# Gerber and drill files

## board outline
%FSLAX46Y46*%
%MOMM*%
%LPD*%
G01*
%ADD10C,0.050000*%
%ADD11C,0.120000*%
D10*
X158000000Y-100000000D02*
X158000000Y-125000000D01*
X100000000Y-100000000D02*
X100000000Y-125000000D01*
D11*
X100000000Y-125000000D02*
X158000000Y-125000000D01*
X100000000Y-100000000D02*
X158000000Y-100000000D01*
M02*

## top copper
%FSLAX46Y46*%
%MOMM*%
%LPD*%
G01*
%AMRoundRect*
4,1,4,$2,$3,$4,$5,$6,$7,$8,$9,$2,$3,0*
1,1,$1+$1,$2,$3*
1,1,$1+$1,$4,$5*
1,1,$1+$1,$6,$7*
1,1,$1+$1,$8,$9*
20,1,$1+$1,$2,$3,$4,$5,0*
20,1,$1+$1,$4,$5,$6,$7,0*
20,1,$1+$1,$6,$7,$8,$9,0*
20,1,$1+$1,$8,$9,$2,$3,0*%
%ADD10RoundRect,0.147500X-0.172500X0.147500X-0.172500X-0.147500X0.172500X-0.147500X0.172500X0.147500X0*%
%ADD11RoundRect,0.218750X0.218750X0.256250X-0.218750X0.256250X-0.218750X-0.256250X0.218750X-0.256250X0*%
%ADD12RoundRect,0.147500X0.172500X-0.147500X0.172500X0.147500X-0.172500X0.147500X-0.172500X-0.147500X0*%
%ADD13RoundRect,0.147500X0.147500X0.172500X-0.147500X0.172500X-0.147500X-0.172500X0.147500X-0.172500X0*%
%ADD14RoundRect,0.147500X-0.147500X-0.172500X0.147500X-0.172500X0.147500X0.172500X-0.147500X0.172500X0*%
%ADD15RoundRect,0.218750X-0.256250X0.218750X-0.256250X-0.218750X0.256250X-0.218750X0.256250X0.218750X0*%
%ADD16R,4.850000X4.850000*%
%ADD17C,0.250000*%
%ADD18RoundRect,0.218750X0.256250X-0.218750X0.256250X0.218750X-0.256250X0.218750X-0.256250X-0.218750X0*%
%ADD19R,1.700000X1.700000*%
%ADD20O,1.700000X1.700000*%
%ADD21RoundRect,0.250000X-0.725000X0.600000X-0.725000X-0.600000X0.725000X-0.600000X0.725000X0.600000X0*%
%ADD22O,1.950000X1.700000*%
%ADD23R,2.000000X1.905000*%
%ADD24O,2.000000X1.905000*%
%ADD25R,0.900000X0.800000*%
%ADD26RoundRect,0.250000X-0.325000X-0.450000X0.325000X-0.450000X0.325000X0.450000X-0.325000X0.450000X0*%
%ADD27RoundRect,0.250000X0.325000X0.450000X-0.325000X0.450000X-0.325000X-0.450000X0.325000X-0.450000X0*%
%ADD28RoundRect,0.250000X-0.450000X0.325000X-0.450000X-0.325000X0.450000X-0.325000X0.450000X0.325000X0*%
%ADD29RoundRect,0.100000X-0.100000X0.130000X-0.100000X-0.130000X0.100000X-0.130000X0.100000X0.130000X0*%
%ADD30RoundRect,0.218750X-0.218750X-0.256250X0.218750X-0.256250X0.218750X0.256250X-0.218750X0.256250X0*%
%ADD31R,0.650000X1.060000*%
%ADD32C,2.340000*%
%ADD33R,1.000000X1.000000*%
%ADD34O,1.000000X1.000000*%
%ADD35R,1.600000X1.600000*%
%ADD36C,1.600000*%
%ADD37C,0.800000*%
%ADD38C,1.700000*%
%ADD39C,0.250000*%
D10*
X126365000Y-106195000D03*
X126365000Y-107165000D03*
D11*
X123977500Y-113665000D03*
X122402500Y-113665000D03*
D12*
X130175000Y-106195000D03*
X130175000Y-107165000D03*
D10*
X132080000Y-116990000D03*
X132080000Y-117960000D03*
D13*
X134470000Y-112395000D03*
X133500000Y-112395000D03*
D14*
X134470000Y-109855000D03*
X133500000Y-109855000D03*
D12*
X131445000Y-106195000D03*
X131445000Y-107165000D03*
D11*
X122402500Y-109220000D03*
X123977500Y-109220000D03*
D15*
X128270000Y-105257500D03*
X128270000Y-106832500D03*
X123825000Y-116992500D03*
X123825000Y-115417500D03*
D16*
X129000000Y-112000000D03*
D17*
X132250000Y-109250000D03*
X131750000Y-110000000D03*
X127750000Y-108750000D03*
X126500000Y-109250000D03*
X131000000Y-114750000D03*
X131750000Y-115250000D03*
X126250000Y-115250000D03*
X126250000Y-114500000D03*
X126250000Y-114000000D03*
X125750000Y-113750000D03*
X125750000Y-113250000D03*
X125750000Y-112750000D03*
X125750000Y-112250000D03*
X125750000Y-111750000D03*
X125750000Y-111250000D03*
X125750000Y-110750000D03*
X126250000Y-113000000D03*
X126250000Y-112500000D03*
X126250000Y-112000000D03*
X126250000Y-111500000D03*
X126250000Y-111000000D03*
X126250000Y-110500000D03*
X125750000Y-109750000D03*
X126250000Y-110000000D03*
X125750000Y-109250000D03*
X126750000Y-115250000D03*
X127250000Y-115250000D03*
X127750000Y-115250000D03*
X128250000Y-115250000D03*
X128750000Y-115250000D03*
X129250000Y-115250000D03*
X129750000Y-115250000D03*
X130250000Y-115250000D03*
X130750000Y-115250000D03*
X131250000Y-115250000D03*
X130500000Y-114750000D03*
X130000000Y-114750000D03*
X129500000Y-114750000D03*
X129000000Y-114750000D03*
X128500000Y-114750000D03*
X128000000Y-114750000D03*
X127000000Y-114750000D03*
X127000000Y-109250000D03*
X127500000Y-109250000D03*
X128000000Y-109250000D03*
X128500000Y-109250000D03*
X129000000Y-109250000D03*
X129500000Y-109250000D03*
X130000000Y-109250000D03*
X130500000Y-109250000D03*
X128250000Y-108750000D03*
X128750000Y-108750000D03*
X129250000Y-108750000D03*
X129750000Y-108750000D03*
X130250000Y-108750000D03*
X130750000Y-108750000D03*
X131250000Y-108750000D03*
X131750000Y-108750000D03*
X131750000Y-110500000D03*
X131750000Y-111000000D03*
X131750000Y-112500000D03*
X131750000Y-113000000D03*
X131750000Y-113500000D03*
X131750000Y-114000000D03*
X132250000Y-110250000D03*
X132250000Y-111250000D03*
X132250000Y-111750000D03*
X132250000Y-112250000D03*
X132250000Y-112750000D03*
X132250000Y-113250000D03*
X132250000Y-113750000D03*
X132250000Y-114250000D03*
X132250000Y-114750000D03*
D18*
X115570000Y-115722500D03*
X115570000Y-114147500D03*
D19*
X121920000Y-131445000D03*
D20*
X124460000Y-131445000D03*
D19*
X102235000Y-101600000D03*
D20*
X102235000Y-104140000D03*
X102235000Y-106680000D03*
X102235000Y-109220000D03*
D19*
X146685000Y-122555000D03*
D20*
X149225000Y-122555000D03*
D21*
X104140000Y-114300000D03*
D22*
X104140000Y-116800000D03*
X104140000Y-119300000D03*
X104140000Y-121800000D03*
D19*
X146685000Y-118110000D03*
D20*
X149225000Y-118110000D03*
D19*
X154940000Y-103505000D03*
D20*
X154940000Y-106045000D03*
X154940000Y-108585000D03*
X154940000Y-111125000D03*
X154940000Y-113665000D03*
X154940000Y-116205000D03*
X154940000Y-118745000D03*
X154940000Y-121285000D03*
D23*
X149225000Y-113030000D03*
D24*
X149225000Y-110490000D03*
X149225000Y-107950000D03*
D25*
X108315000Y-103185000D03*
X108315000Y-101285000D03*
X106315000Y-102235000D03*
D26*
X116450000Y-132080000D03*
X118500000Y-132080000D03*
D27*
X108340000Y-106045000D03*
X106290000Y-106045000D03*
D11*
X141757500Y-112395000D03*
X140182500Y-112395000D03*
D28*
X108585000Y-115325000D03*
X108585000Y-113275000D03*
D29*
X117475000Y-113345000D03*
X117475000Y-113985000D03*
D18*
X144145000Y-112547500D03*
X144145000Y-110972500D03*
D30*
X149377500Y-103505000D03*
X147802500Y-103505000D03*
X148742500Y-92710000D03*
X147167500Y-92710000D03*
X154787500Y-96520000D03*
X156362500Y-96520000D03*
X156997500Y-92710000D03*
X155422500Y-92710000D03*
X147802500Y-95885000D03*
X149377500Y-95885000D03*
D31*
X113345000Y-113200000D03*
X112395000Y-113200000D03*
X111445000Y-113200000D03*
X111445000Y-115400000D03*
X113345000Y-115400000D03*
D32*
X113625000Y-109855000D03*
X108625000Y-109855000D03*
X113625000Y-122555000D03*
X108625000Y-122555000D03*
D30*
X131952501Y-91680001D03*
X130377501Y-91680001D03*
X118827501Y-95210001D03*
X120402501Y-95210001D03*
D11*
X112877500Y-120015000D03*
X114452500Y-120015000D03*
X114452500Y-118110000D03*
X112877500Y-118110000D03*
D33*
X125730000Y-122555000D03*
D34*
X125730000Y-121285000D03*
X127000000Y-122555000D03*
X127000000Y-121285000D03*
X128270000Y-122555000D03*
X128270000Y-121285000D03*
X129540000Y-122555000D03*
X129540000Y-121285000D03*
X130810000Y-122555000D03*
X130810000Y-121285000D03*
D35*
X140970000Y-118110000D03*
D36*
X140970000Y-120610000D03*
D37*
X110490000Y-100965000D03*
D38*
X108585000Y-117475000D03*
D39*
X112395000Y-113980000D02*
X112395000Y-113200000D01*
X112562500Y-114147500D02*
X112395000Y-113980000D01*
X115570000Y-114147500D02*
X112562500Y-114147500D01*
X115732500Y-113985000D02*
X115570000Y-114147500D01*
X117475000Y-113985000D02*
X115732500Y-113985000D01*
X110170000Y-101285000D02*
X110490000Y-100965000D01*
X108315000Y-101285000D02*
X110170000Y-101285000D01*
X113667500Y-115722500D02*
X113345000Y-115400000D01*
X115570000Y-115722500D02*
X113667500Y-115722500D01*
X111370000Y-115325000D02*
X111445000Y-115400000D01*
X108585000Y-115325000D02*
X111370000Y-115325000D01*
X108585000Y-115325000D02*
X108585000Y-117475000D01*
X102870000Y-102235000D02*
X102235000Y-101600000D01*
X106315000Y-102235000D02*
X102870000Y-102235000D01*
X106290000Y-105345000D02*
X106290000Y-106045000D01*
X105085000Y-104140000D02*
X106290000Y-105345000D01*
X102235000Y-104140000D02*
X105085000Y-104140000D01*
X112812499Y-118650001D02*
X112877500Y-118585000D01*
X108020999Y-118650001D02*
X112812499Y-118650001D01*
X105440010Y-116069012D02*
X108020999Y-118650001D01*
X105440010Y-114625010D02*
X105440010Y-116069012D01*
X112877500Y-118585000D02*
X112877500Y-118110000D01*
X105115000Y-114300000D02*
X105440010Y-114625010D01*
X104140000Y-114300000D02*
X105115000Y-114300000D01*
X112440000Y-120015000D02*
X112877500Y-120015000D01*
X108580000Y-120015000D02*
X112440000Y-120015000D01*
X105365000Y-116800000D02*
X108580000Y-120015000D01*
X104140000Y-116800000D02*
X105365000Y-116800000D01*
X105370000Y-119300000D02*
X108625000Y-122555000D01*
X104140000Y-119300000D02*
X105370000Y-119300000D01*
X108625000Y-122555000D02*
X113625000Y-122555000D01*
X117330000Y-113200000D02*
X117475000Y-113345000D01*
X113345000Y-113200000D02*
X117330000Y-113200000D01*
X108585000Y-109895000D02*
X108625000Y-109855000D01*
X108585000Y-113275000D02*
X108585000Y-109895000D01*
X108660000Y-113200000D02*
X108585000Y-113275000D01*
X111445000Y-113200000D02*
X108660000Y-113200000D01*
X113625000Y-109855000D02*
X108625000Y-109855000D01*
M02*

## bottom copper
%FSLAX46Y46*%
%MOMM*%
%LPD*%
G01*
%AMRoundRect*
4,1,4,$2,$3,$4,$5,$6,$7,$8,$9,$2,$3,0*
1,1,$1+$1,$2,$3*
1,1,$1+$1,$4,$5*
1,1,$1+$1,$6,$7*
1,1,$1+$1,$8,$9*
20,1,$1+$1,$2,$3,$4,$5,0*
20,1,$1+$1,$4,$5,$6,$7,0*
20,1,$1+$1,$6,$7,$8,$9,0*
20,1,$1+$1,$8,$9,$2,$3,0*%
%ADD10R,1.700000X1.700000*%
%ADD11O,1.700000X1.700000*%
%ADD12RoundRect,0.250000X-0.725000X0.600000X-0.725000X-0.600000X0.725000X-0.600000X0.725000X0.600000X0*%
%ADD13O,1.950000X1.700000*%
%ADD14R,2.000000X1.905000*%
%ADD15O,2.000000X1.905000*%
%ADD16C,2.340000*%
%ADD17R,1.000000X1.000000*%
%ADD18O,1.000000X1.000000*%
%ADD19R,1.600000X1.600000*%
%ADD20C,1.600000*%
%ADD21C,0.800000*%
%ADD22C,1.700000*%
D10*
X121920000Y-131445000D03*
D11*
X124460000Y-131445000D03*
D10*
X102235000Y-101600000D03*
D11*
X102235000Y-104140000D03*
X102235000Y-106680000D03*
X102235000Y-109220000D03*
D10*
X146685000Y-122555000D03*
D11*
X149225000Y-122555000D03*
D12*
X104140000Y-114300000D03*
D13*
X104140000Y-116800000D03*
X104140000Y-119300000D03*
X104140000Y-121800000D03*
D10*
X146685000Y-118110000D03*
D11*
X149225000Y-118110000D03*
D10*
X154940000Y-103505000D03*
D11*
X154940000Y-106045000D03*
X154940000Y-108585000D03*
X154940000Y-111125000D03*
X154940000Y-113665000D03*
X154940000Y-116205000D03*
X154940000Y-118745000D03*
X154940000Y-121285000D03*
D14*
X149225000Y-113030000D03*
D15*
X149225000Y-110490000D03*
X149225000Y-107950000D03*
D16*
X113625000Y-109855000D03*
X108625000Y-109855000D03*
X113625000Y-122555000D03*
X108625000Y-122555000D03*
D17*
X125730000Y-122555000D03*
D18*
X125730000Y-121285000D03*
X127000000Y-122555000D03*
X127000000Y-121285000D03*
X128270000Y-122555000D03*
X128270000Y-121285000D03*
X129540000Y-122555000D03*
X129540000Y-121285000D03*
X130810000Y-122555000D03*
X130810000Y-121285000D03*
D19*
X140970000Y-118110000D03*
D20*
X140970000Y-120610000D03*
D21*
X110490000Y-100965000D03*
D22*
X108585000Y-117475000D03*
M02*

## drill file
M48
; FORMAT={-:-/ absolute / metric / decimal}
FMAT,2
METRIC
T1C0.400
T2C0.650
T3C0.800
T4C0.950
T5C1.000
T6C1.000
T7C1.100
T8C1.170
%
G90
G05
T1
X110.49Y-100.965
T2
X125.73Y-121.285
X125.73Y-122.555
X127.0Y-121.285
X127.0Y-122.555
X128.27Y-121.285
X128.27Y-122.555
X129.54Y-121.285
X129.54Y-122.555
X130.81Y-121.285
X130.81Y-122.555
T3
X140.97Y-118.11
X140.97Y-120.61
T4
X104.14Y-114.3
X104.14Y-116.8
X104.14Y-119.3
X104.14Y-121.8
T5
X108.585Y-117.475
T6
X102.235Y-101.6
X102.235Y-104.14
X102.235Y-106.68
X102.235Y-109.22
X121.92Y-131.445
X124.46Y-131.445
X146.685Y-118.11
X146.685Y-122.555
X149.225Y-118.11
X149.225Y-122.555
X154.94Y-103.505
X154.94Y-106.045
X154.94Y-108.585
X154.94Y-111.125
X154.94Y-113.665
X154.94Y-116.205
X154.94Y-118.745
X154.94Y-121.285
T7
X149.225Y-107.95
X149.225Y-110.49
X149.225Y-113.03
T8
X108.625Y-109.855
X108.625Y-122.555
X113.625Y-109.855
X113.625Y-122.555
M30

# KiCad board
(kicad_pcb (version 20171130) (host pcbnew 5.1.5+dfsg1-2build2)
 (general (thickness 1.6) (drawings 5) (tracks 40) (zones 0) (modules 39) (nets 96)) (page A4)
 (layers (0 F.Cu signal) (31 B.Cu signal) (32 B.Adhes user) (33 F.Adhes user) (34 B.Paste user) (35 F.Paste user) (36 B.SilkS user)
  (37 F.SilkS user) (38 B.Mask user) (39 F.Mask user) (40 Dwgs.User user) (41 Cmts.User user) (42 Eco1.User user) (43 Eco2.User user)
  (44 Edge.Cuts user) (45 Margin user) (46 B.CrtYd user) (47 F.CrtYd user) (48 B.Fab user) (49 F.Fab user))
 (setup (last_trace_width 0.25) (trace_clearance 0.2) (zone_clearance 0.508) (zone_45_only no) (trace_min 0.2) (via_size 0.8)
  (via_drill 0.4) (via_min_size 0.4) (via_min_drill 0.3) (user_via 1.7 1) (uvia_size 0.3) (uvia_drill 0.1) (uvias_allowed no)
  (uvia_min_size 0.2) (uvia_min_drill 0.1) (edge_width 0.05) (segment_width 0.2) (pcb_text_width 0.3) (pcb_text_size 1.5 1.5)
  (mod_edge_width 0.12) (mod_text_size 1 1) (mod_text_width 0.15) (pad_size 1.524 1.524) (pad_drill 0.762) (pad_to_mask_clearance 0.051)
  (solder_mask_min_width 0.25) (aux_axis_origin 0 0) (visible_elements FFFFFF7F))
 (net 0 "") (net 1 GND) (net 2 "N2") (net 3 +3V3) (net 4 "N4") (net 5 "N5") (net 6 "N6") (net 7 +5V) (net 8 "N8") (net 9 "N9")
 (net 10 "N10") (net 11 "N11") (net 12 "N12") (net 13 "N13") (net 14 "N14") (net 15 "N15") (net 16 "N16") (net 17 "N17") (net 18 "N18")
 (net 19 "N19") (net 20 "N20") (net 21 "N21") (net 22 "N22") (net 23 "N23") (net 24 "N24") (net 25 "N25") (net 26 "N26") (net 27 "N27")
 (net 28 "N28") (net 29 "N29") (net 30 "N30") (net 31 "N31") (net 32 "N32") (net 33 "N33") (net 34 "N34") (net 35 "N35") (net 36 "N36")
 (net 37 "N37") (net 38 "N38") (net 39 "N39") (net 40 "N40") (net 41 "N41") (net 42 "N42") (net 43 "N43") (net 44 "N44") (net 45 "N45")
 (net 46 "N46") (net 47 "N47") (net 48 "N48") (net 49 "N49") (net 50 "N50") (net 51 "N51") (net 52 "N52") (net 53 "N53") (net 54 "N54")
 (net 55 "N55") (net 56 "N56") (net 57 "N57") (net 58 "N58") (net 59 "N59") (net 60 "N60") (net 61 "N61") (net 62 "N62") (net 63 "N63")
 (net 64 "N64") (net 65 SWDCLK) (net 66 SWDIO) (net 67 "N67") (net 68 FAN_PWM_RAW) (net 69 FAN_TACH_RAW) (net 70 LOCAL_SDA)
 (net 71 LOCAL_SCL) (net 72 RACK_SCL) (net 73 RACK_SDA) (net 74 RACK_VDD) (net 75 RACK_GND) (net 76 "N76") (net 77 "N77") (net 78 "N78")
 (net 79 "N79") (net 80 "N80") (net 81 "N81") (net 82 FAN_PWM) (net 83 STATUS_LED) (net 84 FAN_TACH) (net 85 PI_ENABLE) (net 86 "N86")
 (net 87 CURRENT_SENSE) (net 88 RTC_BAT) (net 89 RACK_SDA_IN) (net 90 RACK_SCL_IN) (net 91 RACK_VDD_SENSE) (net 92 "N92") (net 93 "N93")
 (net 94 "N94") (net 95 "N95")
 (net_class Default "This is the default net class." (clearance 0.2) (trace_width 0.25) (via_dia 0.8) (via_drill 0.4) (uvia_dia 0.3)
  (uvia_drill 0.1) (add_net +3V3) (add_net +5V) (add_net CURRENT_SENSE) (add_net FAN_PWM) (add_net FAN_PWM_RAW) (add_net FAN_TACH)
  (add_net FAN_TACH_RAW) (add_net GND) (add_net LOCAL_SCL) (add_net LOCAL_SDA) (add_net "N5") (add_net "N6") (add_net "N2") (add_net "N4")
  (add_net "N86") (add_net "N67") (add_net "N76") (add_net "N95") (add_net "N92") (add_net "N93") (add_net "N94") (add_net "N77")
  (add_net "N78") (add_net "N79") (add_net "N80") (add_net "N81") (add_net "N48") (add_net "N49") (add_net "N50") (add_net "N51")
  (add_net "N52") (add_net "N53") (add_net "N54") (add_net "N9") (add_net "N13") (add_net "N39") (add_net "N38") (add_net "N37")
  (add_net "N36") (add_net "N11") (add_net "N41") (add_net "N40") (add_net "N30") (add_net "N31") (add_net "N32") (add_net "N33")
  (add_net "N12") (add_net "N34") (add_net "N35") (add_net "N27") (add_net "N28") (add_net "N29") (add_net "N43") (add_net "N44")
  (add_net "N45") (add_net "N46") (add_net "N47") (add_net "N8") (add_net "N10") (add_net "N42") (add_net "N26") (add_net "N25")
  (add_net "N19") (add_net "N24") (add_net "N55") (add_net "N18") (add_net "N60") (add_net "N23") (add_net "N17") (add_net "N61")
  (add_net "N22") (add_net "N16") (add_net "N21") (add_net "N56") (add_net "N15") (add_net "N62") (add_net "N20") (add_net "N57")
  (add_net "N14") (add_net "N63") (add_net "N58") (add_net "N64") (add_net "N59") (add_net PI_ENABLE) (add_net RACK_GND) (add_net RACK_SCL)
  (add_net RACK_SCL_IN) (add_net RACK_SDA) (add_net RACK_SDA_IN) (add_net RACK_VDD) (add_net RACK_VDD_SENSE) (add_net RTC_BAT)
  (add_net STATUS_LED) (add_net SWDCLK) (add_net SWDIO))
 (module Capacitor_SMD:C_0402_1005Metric (layer F.Cu) (at 126.365 106.68 270)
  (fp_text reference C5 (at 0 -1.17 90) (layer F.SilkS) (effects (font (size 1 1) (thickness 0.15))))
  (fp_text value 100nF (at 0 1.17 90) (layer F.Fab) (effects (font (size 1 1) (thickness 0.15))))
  (pad 1 smd roundrect (at -0.485 0 270) (size 0.59 0.64) (layers F.Cu F.Paste F.Mask) (roundrect_rratio 0.25) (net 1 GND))
  (pad 2 smd roundrect (at 0.485 0 270) (size 0.59 0.64) (layers F.Cu F.Paste F.Mask) (roundrect_rratio 0.25) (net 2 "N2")))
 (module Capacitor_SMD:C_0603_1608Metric (layer F.Cu) (at 123.19 113.665 180)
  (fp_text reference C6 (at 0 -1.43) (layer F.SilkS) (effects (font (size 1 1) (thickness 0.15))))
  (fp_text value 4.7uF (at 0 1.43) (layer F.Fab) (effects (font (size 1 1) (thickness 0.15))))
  (pad 1 smd roundrect (at -0.7875 0 180) (size 0.875 0.95) (layers F.Cu F.Paste F.Mask) (roundrect_rratio 0.25) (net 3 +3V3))
  (pad 2 smd roundrect (at 0.7875 0 180) (size 0.875 0.95) (layers F.Cu F.Paste F.Mask) (roundrect_rratio 0.25) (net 1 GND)))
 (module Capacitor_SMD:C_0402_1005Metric (layer F.Cu) (at 130.175 106.68 90)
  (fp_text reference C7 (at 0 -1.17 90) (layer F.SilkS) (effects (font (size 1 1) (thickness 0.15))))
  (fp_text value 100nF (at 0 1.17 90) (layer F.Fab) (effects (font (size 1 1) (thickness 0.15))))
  (pad 2 smd roundrect (at 0.485 0 90) (size 0.59 0.64) (layers F.Cu F.Paste F.Mask) (roundrect_rratio 0.25) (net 1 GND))
  (pad 1 smd roundrect (at -0.485 0 90) (size 0.59 0.64) (layers F.Cu F.Paste F.Mask) (roundrect_rratio 0.25) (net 3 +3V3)))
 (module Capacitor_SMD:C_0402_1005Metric (layer F.Cu) (at 132.08 117.475 270)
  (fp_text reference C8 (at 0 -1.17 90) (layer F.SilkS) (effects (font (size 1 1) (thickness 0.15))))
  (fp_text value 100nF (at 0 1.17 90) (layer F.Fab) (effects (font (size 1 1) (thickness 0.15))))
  (pad 1 smd roundrect (at -0.485 0 270) (size 0.59 0.64) (layers F.Cu F.Paste F.Mask) (roundrect_rratio 0.25) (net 3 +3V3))
  (pad 2 smd roundrect (at 0.485 0 270) (size 0.59 0.64) (layers F.Cu F.Paste F.Mask) (roundrect_rratio 0.25) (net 1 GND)))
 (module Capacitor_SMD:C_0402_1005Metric (layer F.Cu) (at 133.985 112.395 180)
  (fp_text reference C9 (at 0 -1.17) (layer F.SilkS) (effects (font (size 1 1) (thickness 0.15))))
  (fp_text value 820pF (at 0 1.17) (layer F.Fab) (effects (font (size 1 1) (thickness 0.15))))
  (pad 1 smd roundrect (at -0.485 0 180) (size 0.59 0.64) (layers F.Cu F.Paste F.Mask) (roundrect_rratio 0.25) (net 1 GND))
  (pad 2 smd roundrect (at 0.485 0 180) (size 0.59 0.64) (layers F.Cu F.Paste F.Mask) (roundrect_rratio 0.25) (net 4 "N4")))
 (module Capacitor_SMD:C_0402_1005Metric (layer F.Cu) (at 133.985 109.855)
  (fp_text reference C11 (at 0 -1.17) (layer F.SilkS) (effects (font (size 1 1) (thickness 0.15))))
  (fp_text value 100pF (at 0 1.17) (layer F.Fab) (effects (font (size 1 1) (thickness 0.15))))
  (pad 2 smd roundrect (at 0.485 0) (size 0.59 0.64) (layers F.Cu F.Paste F.Mask) (roundrect_rratio 0.25) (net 1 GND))
  (pad 1 smd roundrect (at -0.485 0) (size 0.59 0.64) (layers F.Cu F.Paste F.Mask) (roundrect_rratio 0.25) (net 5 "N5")))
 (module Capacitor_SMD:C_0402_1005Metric (layer F.Cu) (at 131.445 106.68 90)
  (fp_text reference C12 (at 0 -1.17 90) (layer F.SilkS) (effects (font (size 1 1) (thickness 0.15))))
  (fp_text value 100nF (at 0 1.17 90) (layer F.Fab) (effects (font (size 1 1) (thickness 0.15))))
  (pad 2 smd roundrect (at 0.485 0 90) (size 0.59 0.64) (layers F.Cu F.Paste F.Mask) (roundrect_rratio 0.25) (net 1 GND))
  (pad 1 smd roundrect (at -0.485 0 90) (size 0.59 0.64) (layers F.Cu F.Paste F.Mask) (roundrect_rratio 0.25) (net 3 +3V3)))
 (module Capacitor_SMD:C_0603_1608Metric (layer F.Cu) (at 123.19 109.22 180)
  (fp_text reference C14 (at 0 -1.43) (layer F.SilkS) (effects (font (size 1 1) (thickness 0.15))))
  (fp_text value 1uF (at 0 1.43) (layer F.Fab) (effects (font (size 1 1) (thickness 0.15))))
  (pad 2 smd roundrect (at 0.7875 0 180) (size 0.875 0.95) (layers F.Cu F.Paste F.Mask) (roundrect_rratio 0.25) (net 1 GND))
  (pad 1 smd roundrect (at -0.7875 0 180) (size 0.875 0.95) (layers F.Cu F.Paste F.Mask) (roundrect_rratio 0.25) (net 3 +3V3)))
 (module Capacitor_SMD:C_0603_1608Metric (layer F.Cu) (at 128.27 106.045 270)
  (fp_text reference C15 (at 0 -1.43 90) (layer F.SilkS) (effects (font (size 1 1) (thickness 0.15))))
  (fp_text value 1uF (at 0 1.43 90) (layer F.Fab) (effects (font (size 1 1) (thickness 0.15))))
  (pad 1 smd roundrect (at -0.7875 0 270) (size 0.875 0.95) (layers F.Cu F.Paste F.Mask) (roundrect_rratio 0.25) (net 1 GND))
  (pad 2 smd roundrect (at 0.7875 0 270) (size 0.875 0.95) (layers F.Cu F.Paste F.Mask) (roundrect_rratio 0.25) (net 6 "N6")))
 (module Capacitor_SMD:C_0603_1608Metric (layer F.Cu) (at 123.825 116.205 270)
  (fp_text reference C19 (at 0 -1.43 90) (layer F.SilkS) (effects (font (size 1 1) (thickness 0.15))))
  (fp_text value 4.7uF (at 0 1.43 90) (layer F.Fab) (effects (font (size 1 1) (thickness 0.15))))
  (pad 2 smd roundrect (at 0.7875 0 270) (size 0.875 0.95) (layers F.Cu F.Paste F.Mask) (roundrect_rratio 0.25) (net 1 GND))
  (pad 1 smd roundrect (at -0.7875 0 270) (size 0.875 0.95) (layers F.Cu F.Paste F.Mask) (roundrect_rratio 0.25) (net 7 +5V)))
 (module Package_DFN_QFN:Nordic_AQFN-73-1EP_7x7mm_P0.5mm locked (layer F.Cu) (at 129 112)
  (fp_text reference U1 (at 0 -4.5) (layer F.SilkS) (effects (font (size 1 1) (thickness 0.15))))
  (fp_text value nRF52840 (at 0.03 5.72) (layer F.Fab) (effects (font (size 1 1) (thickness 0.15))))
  (pad "" smd rect (at 1.2125 1.2125 180) (size 2 2) (layers F.Paste))
  (pad "" smd rect (at -1.2125 1.2125 180) (size 2 2) (layers F.Paste))
  (pad "" smd rect (at 1.2125 -1.2125 180) (size 2 2) (layers F.Paste))
  (pad "" smd rect (at -1.2125 -1.2125 180) (size 2 2) (layers F.Paste))
  (pad EP smd rect (at 0 0 180) (size 4.85 4.85) (layers F.Cu F.Mask) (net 1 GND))
  (pad B24 smd circle (at 3.25 -2.75 180) (size 0.25 0.25) (layers F.Cu F.Paste F.Mask) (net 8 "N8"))
  (pad D23 smd circle (at 2.75 -2 180) (size 0.25 0.25) (layers F.Cu F.Paste F.Mask) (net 5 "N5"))
  (pad A8 smd circle (at -1.25 -3.25 180) (size 0.25 0.25) (layers F.Cu F.Paste F.Mask) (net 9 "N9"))
  (pad B3 smd circle (at -2.5 -2.75 180) (size 0.25 0.25) (layers F.Cu F.Paste F.Mask) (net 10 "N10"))
  (pad AC21 smd circle (at 2 2.75 180) (size 0.25 0.25) (layers F.Cu F.Paste F.Mask) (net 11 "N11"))
  (pad AD23 smd circle (at 2.75 3.25 180) (size 0.25 0.25) (layers F.Cu F.Paste F.Mask) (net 3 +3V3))
  (pad AD2 smd circle (at -2.75 3.25 180) (size 0.25 0.25) (layers F.Cu F.Paste F.Mask) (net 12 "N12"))
  (pad AB2 smd circle (at -2.75 2.5 180) (size 0.25 0.25) (layers F.Cu F.Paste F.Mask) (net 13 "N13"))
  (pad Y2 smd circle (at -2.75 2 180) (size 0.25 0.25) (layers F.Cu F.Paste F.Mask) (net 7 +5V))
  (pad W1 smd circle (at -3.25 1.75 180) (size 0.25 0.25) (layers F.Cu F.Paste F.Mask) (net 3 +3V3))
  (pad U1 smd circle (at -3.25 1.25 180) (size 0.25 0.25) (layers F.Cu F.Paste F.Mask) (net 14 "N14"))
  (pad R1 smd circle (at -3.25 0.75 180) (size 0.25 0.25) (layers F.Cu F.Paste F.Mask) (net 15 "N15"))
  (pad N1 smd circle (at -3.25 0.25 180) (size 0.25 0.25) (layers F.Cu F.Paste F.Mask) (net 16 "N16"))
  (pad L1 smd circle (at -3.25 -0.25 180) (size 0.25 0.25) (layers F.Cu F.Paste F.Mask) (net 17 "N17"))
  (pad J1 smd circle (at -3.25 -0.75 180) (size 0.25 0.25) (layers F.Cu F.Paste F.Mask) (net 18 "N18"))
  (pad G1 smd circle (at -3.25 -1.25 180) (size 0.25 0.25) (layers F.Cu F.Paste F.Mask) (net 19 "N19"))
  (pad T2 smd circle (at -2.75 1 180) (size 0.25 0.25) (layers F.Cu F.Paste F.Mask) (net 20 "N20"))
  (pad P2 smd circle (at -2.75 0.5 180) (size 0.25 0.25) (layers F.Cu F.Paste F.Mask) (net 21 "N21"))
  (pad M2 smd circle (at -2.75 0 180) (size 0.25 0.25) (layers F.Cu F.Paste F.Mask) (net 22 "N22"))
  (pad K2 smd circle (at -2.75 -0.5 180) (size 0.25 0.25) (layers F.Cu F.Paste F.Mask) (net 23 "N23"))
  (pad H2 smd circle (at -2.75 -1 180) (size 0.25 0.25) (layers F.Cu F.Paste F.Mask) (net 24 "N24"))
  (pad F2 smd circle (at -2.75 -1.5 180) (size 0.25 0.25) (layers F.Cu F.Paste F.Mask) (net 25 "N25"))
  (pad C1 smd circle (at -3.25 -2.25 180) (size 0.25 0.25) (layers F.Cu F.Paste F.Mask) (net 2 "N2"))
  (pad D2 smd circle (at -2.75 -2 180) (size 0.25 0.25) (layers F.Cu F.Paste F.Mask) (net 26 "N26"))
  (pad B1 smd circle (at -3.25 -2.75 180) (size 0.25 0.25) (layers F.Cu F.Paste F.Mask) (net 3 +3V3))
  (pad AD4 smd circle (at -2.25 3.25 180) (size 0.25 0.25) (layers F.Cu F.Paste F.Mask) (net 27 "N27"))
  (pad AD6 smd circle (at -1.75 3.25 180) (size 0.25 0.25) (layers F.Cu F.Paste F.Mask) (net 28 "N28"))
  (pad AD8 smd circle (at -1.25 3.25 180) (size 0.25 0.25) (layers F.Cu F.Paste F.Mask) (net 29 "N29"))
  (pad AD10 smd circle (at -0.75 3.25 180) (size 0.25 0.25) (layers F.Cu F.Paste F.Mask) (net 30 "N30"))
  (pad AD12 smd circle (at -0.25 3.25 180) (size 0.25 0.25) (layers F.Cu F.Paste F.Mask) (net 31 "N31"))
  (pad AD14 smd circle (at 0.25 3.25 180) (size 0.25 0.25) (layers F.Cu F.Paste F.Mask) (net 3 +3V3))
  (pad AD16 smd circle (at 0.75 3.25 180) (size 0.25 0.25) (layers F.Cu F.Paste F.Mask) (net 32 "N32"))
  (pad AD18 smd circle (at 1.25 3.25 180) (size 0.25 0.25) (layers F.Cu F.Paste F.Mask) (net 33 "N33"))
  (pad AD20 smd circle (at 1.75 3.25 180) (size 0.25 0.25) (layers F.Cu F.Paste F.Mask) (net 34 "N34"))
  (pad AD22 smd circle (at 2.25 3.25 180) (size 0.25 0.25) (layers F.Cu F.Paste F.Mask) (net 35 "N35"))
  (pad AC19 smd circle (at 1.5 2.75 180) (size 0.25 0.25) (layers F.Cu F.Paste F.Mask) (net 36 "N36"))
  (pad AC17 smd circle (at 1 2.75 180) (size 0.25 0.25) (layers F.Cu F.Paste F.Mask) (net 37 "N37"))
  (pad AC15 smd circle (at 0.5 2.75 180) (size 0.25 0.25) (layers F.Cu F.Paste F.Mask) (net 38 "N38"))
  (pad AC13 smd circle (at 0 2.75 180) (size 0.25 0.25) (layers F.Cu F.Paste F.Mask) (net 3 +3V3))
  (pad AC11 smd circle (at -0.5 2.75 180) (size 0.25 0.25) (layers F.Cu F.Paste F.Mask) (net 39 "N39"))
  (pad AC9 smd circle (at -1 2.75 180) (size 0.25 0.25) (layers F.Cu F.Paste F.Mask) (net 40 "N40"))
  (pad AC5 smd circle (at -2 2.75 180) (size 0.25 0.25) (layers F.Cu F.Paste F.Mask) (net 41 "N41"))
  (pad B5 smd circle (at -2 -2.75 180) (size 0.25 0.25) (layers F.Cu F.Paste F.Mask) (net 6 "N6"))
  (pad B7 smd circle (at -1.5 -2.75 180) (size 0.25 0.25) (layers F.Cu F.Paste F.Mask) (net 1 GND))
  (pad B9 smd circle (at -1 -2.75 180) (size 0.25 0.25) (layers F.Cu F.Paste F.Mask) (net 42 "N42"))
  (pad B11 smd circle (at -0.5 -2.75 180) (size 0.25 0.25) (layers F.Cu F.Paste F.Mask) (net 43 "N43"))
  (pad B13 smd circle (at 0 -2.75 180) (size 0.25 0.25) (layers F.Cu F.Paste F.Mask) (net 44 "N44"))
  (pad B15 smd circle (at 0.5 -2.75 180) (size 0.25 0.25) (layers F.Cu F.Paste F.Mask) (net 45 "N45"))
  (pad B17 smd circle (at 1 -2.75 180) (size 0.25 0.25) (layers F.Cu F.Paste F.Mask) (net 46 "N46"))
  (pad B19 smd circle (at 1.5 -2.75 180) (size 0.25 0.25) (layers F.Cu F.Paste F.Mask) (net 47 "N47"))
  (pad A10 smd circle (at -0.75 -3.25 180) (size 0.25 0.25) (layers F.Cu F.Paste F.Mask) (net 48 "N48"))
  (pad A12 smd circle (at -0.25 -3.25 180) (size 0.25 0.25) (layers F.Cu F.Paste F.Mask) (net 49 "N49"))
  (pad A14 smd circle (at 0.25 -3.25 180) (size 0.25 0.25) (layers F.Cu F.Paste F.Mask) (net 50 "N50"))
  (pad A16 smd circle (at 0.75 -3.25 180) (size 0.25 0.25) (layers F.Cu F.Paste F.Mask) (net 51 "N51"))
  (pad A18 smd circle (at 1.25 -3.25 180) (size 0.25 0.25) (layers F.Cu F.Paste F.Mask) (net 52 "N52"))
  (pad A20 smd circle (at 1.75 -3.25 180) (size 0.25 0.25) (layers F.Cu F.Paste F.Mask) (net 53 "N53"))
  (pad A22 smd circle (at 2.25 -3.25 180) (size 0.25 0.25) (layers F.Cu F.Paste F.Mask) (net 3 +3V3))
  (pad A23 smd circle (at 2.75 -3.25 180) (size 0.25 0.25) (layers F.Cu F.Paste F.Mask) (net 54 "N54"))
  (pad F23 smd circle (at 2.75 -1.5 180) (size 0.25 0.25) (layers F.Cu F.Paste F.Mask) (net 1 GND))
  (pad H23 smd circle (at 2.75 -1 180) (size 0.25 0.25) (layers F.Cu F.Paste F.Mask) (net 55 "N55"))
  (pad P23 smd circle (at 2.75 0.5 180) (size 0.25 0.25) (layers F.Cu F.Paste F.Mask) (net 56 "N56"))
  (pad T23 smd circle (at 2.75 1 180) (size 0.25 0.25) (layers F.Cu F.Paste F.Mask) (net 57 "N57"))
  (pad V23 smd circle (at 2.75 1.5 180) (size 0.25 0.25) (layers F.Cu F.Paste F.Mask) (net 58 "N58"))
  (pad Y23 smd circle (at 2.75 2 180) (size 0.25 0.25) (layers F.Cu F.Paste F.Mask) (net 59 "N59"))
  (pad E24 smd circle (at 3.25 -1.75 180) (size 0.25 0.25) (layers F.Cu F.Paste F.Mask) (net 6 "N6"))
  (pad J24 smd circle (at 3.25 -0.75 180) (size 0.25 0.25) (layers F.Cu F.Paste F.Mask) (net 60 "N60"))
  (pad L24 smd circle (at 3.25 -0.25 180) (size 0.25 0.25) (layers F.Cu F.Paste F.Mask) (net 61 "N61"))
  (pad N24 smd circle (at 3.25 0.25 180) (size 0.25 0.25) (layers F.Cu F.Paste F.Mask) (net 4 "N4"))
  (pad R24 smd circle (at 3.25 0.75 180) (size 0.25 0.25) (layers F.Cu F.Paste F.Mask) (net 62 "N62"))
  (pad U24 smd circle (at 3.25 1.25 180) (size 0.25 0.25) (layers F.Cu F.Paste F.Mask) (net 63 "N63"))
  (pad W24 smd circle (at 3.25 1.75 180) (size 0.25 0.25) (layers F.Cu F.Paste F.Mask) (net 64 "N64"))
  (pad AA24 smd circle (at 3.25 2.25 180) (size 0.25 0.25) (layers F.Cu F.Paste F.Mask) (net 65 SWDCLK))
  (pad AC24 smd circle (at 3.25 2.75 180) (size 0.25 0.25) (layers F.Cu F.Paste F.Mask) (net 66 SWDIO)))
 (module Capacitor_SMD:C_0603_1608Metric (layer F.Cu) (at 115.57 114.935 90)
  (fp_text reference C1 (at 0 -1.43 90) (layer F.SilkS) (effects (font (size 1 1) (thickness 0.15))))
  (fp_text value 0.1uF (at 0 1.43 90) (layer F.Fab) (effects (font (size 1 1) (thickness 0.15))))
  (pad 1 smd roundrect (at -0.7875 0 90) (size 0.875 0.95) (layers F.Cu F.Paste F.Mask) (roundrect_rratio 0.25) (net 3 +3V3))
  (pad 2 smd roundrect (at 0.7875 0 90) (size 0.875 0.95) (layers F.Cu F.Paste F.Mask) (roundrect_rratio 0.25) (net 1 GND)))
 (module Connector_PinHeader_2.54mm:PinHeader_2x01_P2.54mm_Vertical (layer F.Cu) (at 121.92 131.445)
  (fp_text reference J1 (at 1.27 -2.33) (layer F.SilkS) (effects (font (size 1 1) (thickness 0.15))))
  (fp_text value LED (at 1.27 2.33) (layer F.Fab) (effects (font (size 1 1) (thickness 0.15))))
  (pad 1 thru_hole rect (at 0 0) (size 1.7 1.7) (drill 1) (layers *.Cu *.Mask) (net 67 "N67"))
  (pad 2 thru_hole oval (at 2.54 0) (size 1.7 1.7) (drill 1) (layers *.Cu *.Mask) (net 1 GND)))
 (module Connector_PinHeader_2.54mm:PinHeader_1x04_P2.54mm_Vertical (layer F.Cu) (at 102.235 101.6)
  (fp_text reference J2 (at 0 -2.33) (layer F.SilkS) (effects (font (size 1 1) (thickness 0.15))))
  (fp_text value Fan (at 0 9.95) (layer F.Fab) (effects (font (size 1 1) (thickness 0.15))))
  (pad 1 thru_hole rect (at 0 0) (size 1.7 1.7) (drill 1) (layers *.Cu *.Mask) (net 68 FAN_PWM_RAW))
  (pad 2 thru_hole oval (at 0 2.54) (size 1.7 1.7) (drill 1) (layers *.Cu *.Mask) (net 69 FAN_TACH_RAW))
  (pad 3 thru_hole oval (at 0 5.08) (size 1.7 1.7) (drill 1) (layers *.Cu *.Mask) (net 7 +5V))
  (pad 4 thru_hole oval (at 0 7.62) (size 1.7 1.7) (drill 1) (layers *.Cu *.Mask) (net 1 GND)))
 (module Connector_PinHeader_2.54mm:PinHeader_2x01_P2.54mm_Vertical (layer F.Cu) (at 146.685 122.555)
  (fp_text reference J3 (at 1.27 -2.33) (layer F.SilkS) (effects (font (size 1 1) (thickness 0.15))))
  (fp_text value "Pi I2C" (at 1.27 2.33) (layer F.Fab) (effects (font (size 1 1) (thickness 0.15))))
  (pad 1 thru_hole rect (at 0 0) (size 1.7 1.7) (drill 1) (layers *.Cu *.Mask) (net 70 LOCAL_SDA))
  (pad 2 thru_hole oval (at 2.54 0) (size 1.7 1.7) (drill 1) (layers *.Cu *.Mask) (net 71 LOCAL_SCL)))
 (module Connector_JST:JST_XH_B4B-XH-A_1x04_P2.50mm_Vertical (layer F.Cu) (at 104.14 114.3 270)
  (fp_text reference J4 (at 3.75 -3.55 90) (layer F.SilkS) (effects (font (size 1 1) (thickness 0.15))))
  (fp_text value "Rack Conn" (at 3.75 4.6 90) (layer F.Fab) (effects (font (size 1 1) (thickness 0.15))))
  (pad 1 thru_hole roundrect (at 0 0 270) (size 1.7 1.95) (drill 0.95) (layers *.Cu *.Mask) (roundrect_rratio 0.147059) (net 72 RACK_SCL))
  (pad 2 thru_hole oval (at 2.5 0 270) (size 1.7 1.95) (drill 0.95) (layers *.Cu *.Mask) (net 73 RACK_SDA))
  (pad 3 thru_hole oval (at 5 0 270) (size 1.7 1.95) (drill 0.95) (layers *.Cu *.Mask) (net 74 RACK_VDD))
  (pad 4 thru_hole oval (at 7.5 0 270) (size 1.7 1.95) (drill 0.95) (layers *.Cu *.Mask) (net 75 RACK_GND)))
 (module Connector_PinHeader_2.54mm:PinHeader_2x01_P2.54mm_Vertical (layer F.Cu) (at 146.685 118.11)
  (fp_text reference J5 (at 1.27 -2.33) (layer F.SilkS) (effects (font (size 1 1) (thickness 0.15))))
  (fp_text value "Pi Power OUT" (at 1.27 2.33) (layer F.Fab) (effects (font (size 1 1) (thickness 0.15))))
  (pad 1 thru_hole rect (at 0 0) (size 1.7 1.7) (drill 1) (layers *.Cu *.Mask) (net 7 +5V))
  (pad 2 thru_hole oval (at 2.54 0) (size 1.7 1.7) (drill 1) (layers *.Cu *.Mask) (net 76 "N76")))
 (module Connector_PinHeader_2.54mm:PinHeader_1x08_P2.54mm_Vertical (layer F.Cu) (at 154.94 103.505)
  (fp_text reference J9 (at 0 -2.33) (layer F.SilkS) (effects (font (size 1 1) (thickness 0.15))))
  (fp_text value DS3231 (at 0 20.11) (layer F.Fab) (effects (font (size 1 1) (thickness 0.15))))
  (pad 1 thru_hole rect (at 0 0) (size 1.7 1.7) (drill 1) (layers *.Cu *.Mask) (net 3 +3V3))
  (pad 2 thru_hole oval (at 0 2.54) (size 1.7 1.7) (drill 1) (layers *.Cu *.Mask) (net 1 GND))
  (pad 3 thru_hole oval (at 0 5.08) (size 1.7 1.7) (drill 1) (layers *.Cu *.Mask) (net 71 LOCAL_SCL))
  (pad 4 thru_hole oval (at 0 7.62) (size 1.7 1.7) (drill 1) (layers *.Cu *.Mask) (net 70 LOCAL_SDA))
  (pad 5 thru_hole oval (at 0 10.16) (size 1.7 1.7) (drill 1) (layers *.Cu *.Mask) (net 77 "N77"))
  (pad 6 thru_hole oval (at 0 12.7) (size 1.7 1.7) (drill 1) (layers *.Cu *.Mask) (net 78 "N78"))
  (pad 7 thru_hole oval (at 0 15.24) (size 1.7 1.7) (drill 1) (layers *.Cu *.Mask) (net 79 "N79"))
  (pad 8 thru_hole oval (at 0 17.78) (size 1.7 1.7) (drill 1) (layers *.Cu *.Mask) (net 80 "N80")))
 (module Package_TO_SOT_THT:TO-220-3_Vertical (layer F.Cu) (at 149.225 113.03 90)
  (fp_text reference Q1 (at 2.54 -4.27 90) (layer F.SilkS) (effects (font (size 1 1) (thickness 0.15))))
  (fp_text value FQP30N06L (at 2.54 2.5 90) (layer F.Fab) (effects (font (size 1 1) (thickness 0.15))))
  (pad 1 thru_hole rect (at 0 0 90) (size 1.905 2) (drill 1.1) (layers *.Cu *.Mask) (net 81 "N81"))
  (pad 2 thru_hole oval (at 2.54 0 90) (size 1.905 2) (drill 1.1) (layers *.Cu *.Mask) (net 76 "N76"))
  (pad 3 thru_hole oval (at 5.08 0 90) (size 1.905 2) (drill 1.1) (layers *.Cu *.Mask) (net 1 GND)))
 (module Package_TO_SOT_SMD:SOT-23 (layer F.Cu) (at 107.315 102.235 180)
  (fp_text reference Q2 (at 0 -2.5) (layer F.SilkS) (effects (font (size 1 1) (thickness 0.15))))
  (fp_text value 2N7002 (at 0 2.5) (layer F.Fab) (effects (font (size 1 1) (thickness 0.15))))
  (pad 1 smd rect (at -1 -0.95 180) (size 0.9 0.8) (layers F.Cu F.Paste F.Mask) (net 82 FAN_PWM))
  (pad 2 smd rect (at -1 0.95 180) (size 0.9 0.8) (layers F.Cu F.Paste F.Mask) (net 1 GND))
  (pad 3 smd rect (at 1 0 180) (size 0.9 0.8) (layers F.Cu F.Paste F.Mask) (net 68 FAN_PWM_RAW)))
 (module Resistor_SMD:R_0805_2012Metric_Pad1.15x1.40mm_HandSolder (layer F.Cu) (at 117.475 132.08)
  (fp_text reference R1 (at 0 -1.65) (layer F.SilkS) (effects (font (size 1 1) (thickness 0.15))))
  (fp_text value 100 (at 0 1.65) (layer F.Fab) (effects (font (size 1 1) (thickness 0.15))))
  (pad 1 smd roundrect (at -1.025 0) (size 1.15 1.4) (layers F.Cu F.Paste F.Mask) (roundrect_rratio 0.217391) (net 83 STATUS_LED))
  (pad 2 smd roundrect (at 1.025 0) (size 1.15 1.4) (layers F.Cu F.Paste F.Mask) (roundrect_rratio 0.217391) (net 67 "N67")))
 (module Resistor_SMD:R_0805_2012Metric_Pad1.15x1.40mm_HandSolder (layer F.Cu) (at 107.315 106.045 180)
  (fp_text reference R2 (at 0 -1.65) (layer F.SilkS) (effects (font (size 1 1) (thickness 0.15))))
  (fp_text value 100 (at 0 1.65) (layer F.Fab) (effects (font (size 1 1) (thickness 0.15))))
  (pad 1 smd roundrect (at -1.025 0 180) (size 1.15 1.4) (layers F.Cu F.Paste F.Mask) (roundrect_rratio 0.217391) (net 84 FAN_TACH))
  (pad 2 smd roundrect (at 1.025 0 180) (size 1.15 1.4) (layers F.Cu F.Paste F.Mask) (roundrect_rratio 0.217391) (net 69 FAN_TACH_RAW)))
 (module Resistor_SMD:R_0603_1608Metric (layer F.Cu) (at 140.97 112.395 180)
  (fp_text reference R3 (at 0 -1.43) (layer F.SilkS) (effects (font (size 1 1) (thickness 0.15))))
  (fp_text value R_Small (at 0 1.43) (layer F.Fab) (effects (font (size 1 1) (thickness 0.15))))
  (pad 1 smd roundrect (at -0.7875 0 180) (size 0.875 0.95) (layers F.Cu F.Paste F.Mask) (roundrect_rratio 0.25) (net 81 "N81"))
  (pad 2 smd roundrect (at 0.7875 0 180) (size 0.875 0.95) (layers F.Cu F.Paste F.Mask) (roundrect_rratio 0.25) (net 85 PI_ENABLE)))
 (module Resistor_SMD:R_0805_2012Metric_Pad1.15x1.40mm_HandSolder (layer F.Cu) (at 108.585 114.3 270)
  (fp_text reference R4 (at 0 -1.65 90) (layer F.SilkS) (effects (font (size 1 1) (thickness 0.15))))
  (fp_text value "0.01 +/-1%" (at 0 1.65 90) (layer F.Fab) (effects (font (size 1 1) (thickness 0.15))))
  (pad 2 smd roundrect (at 1.025 0 270) (size 1.15 1.4) (layers F.Cu F.Paste F.Mask) (roundrect_rratio 0.217391) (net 7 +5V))
  (pad 1 smd roundrect (at -1.025 0 270) (size 1.15 1.4) (layers F.Cu F.Paste F.Mask) (roundrect_rratio 0.217391) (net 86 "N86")))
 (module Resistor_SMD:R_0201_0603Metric (layer F.Cu) (at 117.475 113.665 270)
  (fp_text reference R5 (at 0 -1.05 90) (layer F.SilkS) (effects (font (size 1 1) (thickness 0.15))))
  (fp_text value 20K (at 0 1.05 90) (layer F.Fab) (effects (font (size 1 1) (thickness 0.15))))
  (pad "" smd roundrect (at -0.345 0 270) (size 0.318 0.36) (layers F.Paste) (roundrect_rratio 0.25))
  (pad "" smd roundrect (at 0.345 0 270) (size 0.318 0.36) (layers F.Paste) (roundrect_rratio 0.25))
  (pad 1 smd roundrect (at -0.32 0 270) (size 0.46 0.4) (layers F.Cu F.Mask) (roundrect_rratio 0.25) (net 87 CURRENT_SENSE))
  (pad 2 smd roundrect (at 0.32 0 270) (size 0.46 0.4) (layers F.Cu F.Mask) (roundrect_rratio 0.25) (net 1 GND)))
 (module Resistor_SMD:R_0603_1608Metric (layer F.Cu) (at 144.145 111.76 90)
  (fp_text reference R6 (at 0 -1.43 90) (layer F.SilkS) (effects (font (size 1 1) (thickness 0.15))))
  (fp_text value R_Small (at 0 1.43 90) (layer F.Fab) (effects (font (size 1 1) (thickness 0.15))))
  (pad 1 smd roundrect (at -0.7875 0 90) (size 0.875 0.95) (layers F.Cu F.Paste F.Mask) (roundrect_rratio 0.25) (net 81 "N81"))
  (pad 2 smd roundrect (at 0.7875 0 90) (size 0.875 0.95) (layers F.Cu F.Paste F.Mask) (roundrect_rratio 0.25) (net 1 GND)))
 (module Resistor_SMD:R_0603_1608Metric (layer F.Cu) (at 148.59 103.505)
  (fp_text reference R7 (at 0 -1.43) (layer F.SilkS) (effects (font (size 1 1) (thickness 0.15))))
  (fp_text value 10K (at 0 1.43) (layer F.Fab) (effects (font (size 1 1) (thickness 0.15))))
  (pad 2 smd roundrect (at 0.7875 0) (size 0.875 0.95) (layers F.Cu F.Paste F.Mask) (roundrect_rratio 0.25) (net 77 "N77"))
  (pad 1 smd roundrect (at -0.7875 0) (size 0.875 0.95) (layers F.Cu F.Paste F.Mask) (roundrect_rratio 0.25) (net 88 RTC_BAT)))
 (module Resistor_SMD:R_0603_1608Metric (layer F.Cu) (at 147.955 92.71)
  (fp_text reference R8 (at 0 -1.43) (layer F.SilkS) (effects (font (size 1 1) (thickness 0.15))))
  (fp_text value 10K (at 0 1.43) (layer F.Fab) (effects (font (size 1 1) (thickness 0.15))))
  (pad 2 smd roundrect (at 0.7875 0) (size 0.875 0.95) (layers F.Cu F.Paste F.Mask) (roundrect_rratio 0.25) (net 70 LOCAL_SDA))
  (pad 1 smd roundrect (at -0.7875 0) (size 0.875 0.95) (layers F.Cu F.Paste F.Mask) (roundrect_rratio 0.25) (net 3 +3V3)))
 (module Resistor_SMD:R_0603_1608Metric (layer F.Cu) (at 155.575 96.52)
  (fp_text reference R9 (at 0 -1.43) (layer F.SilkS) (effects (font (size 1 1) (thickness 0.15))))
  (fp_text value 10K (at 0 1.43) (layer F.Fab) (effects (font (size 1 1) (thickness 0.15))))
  (pad 1 smd roundrect (at -0.7875 0) (size 0.875 0.95) (layers F.Cu F.Paste F.Mask) (roundrect_rratio 0.25) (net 3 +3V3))
  (pad 2 smd roundrect (at 0.7875 0) (size 0.875 0.95) (layers F.Cu F.Paste F.Mask) (roundrect_rratio 0.25) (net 71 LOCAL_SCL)))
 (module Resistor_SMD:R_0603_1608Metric (layer F.Cu) (at 156.21 92.71)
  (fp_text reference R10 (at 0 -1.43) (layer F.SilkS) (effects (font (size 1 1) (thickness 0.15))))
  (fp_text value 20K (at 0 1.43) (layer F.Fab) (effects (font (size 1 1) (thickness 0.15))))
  (pad 2 smd roundrect (at 0.7875 0) (size 0.875 0.95) (layers F.Cu F.Paste F.Mask) (roundrect_rratio 0.25) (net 3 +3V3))
  (pad 1 smd roundrect (at -0.7875 0) (size 0.875 0.95) (layers F.Cu F.Paste F.Mask) (roundrect_rratio 0.25) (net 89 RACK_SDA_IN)))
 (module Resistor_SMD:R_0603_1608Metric (layer F.Cu) (at 148.59 95.885)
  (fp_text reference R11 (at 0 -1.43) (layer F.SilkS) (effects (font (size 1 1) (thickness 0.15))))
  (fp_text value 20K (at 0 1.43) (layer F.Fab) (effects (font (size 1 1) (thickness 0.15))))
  (pad 1 smd roundrect (at -0.7875 0) (size 0.875 0.95) (layers F.Cu F.Paste F.Mask) (roundrect_rratio 0.25) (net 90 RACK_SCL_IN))
  (pad 2 smd roundrect (at 0.7875 0) (size 0.875 0.95) (layers F.Cu F.Paste F.Mask) (roundrect_rratio 0.25) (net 3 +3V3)))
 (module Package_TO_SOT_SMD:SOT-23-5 (layer F.Cu) (at 112.395 114.3 270)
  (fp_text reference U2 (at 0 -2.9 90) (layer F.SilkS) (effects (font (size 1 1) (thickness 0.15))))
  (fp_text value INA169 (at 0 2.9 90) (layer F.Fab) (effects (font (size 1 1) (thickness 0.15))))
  (pad 1 smd rect (at -1.1 -0.95 270) (size 1.06 0.65) (layers F.Cu F.Paste F.Mask) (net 87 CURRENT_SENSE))
  (pad 2 smd rect (at -1.1 0 270) (size 1.06 0.65) (layers F.Cu F.Paste F.Mask) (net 1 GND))
  (pad 3 smd rect (at -1.1 0.95 270) (size 1.06 0.65) (layers F.Cu F.Paste F.Mask) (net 86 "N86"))
  (pad 4 smd rect (at 1.1 0.95 270) (size 1.06 0.65) (layers F.Cu F.Paste F.Mask) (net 7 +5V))
  (pad 5 smd rect (at 1.1 -0.95 270) (size 1.06 0.65) (layers F.Cu F.Paste F.Mask) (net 3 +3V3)))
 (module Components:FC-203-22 (layer F.Cu) (at 111.125 116.205 270)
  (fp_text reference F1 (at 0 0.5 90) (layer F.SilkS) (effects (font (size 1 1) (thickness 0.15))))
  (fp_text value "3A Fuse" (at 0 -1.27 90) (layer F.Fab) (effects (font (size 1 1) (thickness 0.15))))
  (pad 1 thru_hole circle (at -6.35 -2.5 270) (size 2.34 2.34) (drill 1.17) (layers *.Cu *.Mask) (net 86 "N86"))
  (pad 1 thru_hole circle (at -6.35 2.5 270) (size 2.34 2.34) (drill 1.17) (layers *.Cu *.Mask) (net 86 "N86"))
  (pad 2 thru_hole circle (at 6.35 -2.5 270) (size 2.34 2.34) (drill 1.17) (layers *.Cu *.Mask) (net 74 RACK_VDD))
  (pad 2 thru_hole circle (at 6.35 2.5 270) (size 2.34 2.34) (drill 1.17) (layers *.Cu *.Mask) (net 74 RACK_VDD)))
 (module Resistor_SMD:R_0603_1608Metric (layer F.Cu) (at 131.165001 91.680001)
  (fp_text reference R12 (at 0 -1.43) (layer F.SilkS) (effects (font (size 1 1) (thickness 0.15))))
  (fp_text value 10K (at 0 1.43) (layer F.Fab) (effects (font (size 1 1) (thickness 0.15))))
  (pad 2 smd roundrect (at 0.7875 0) (size 0.875 0.95) (layers F.Cu F.Paste F.Mask) (roundrect_rratio 0.25) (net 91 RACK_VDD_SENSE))
  (pad 1 smd roundrect (at -0.7875 0) (size 0.875 0.95) (layers F.Cu F.Paste F.Mask) (roundrect_rratio 0.25) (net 74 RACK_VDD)))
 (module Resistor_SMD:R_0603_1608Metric (layer F.Cu) (at 119.615001 95.210001)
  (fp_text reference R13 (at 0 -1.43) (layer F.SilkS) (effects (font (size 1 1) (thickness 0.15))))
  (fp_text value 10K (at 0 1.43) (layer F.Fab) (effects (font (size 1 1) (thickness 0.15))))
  (pad 1 smd roundrect (at -0.7875 0) (size 0.875 0.95) (layers F.Cu F.Paste F.Mask) (roundrect_rratio 0.25) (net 91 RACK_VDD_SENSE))
  (pad 2 smd roundrect (at 0.7875 0) (size 0.875 0.95) (layers F.Cu F.Paste F.Mask) (roundrect_rratio 0.25) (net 1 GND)))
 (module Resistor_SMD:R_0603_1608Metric (layer F.Cu) (at 113.665 120.015 180)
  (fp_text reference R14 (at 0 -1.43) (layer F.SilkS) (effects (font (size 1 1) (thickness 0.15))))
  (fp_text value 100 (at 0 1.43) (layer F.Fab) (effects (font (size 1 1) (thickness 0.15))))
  (pad 2 smd roundrect (at 0.7875 0 180) (size 0.875 0.95) (layers F.Cu F.Paste F.Mask) (roundrect_rratio 0.25) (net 73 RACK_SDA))
  (pad 1 smd roundrect (at -0.7875 0 180) (size 0.875 0.95) (layers F.Cu F.Paste F.Mask) (roundrect_rratio 0.25) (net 89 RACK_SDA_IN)))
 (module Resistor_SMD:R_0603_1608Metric (layer F.Cu) (at 113.665 118.11 180)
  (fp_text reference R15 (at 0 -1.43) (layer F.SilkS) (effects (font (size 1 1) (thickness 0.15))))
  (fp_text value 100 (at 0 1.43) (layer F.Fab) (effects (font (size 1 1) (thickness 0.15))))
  (pad 1 smd roundrect (at -0.7875 0 180) (size 0.875 0.95) (layers F.Cu F.Paste F.Mask) (roundrect_rratio 0.25) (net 90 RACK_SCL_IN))
  (pad 2 smd roundrect (at 0.7875 0 180) (size 0.875 0.95) (layers F.Cu F.Paste F.Mask) (roundrect_rratio 0.25) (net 72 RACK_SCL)))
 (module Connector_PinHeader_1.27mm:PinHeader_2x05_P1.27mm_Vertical (layer F.Cu) (at 125.73 122.555 90)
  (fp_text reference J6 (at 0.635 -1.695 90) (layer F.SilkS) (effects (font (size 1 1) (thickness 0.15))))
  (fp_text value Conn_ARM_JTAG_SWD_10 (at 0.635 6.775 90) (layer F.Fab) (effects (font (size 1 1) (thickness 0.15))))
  (pad 1 thru_hole rect (at 0 0 90) (size 1 1) (drill 0.65) (layers *.Cu *.Mask) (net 3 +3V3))
  (pad 2 thru_hole oval (at 1.27 0 90) (size 1 1) (drill 0.65) (layers *.Cu *.Mask) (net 66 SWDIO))
  (pad 3 thru_hole oval (at 0 1.27 90) (size 1 1) (drill 0.65) (layers *.Cu *.Mask) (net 1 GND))
  (pad 4 thru_hole oval (at 1.27 1.27 90) (size 1 1) (drill 0.65) (layers *.Cu *.Mask) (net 65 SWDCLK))
  (pad 5 thru_hole oval (at 0 2.54 90) (size 1 1) (drill 0.65) (layers *.Cu *.Mask) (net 1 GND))
  (pad 6 thru_hole oval (at 1.27 2.54 90) (size 1 1) (drill 0.65) (layers *.Cu *.Mask) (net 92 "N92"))
  (pad 7 thru_hole oval (at 0 3.81 90) (size 1 1) (drill 0.65) (layers *.Cu *.Mask) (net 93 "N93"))
  (pad 8 thru_hole oval (at 1.27 3.81 90) (size 1 1) (drill 0.65) (layers *.Cu *.Mask) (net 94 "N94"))
  (pad 9 thru_hole oval (at 0 5.08 90) (size 1 1) (drill 0.65) (layers *.Cu *.Mask) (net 1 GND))
  (pad 10 thru_hole oval (at 1.27 5.08 90) (size 1 1) (drill 0.65) (layers *.Cu *.Mask) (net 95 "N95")))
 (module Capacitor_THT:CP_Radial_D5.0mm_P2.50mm (layer F.Cu) (at 140.97 118.11 270)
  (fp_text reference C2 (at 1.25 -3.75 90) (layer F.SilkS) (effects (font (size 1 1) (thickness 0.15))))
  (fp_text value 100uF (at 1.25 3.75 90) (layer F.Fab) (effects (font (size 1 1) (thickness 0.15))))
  (pad 1 thru_hole rect (at 0 0 270) (size 1.6 1.6) (drill 0.8) (layers *.Cu *.Mask) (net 7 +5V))
  (pad 2 thru_hole circle (at 2.5 0 270) (size 1.6 1.6) (drill 0.8) (layers *.Cu *.Mask) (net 1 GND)))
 (gr_line (start 158 100) (end 158 125) (layer Edge.Cuts) (width 0.05))
 (gr_line (start 100 100) (end 100 125) (layer Edge.Cuts) (width 0.05))
 (gr_line (start 100 125) (end 158 125) (layer Edge.Cuts) (width 0.12))
 (gr_line (start 100 100) (end 158 100) (layer Edge.Cuts) (width 0.12))
 (via (at 110.49 100.965) (size 0.8) (drill 0.4) (layers F.Cu B.Cu) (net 1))
 (segment (start 112.395 113.98) (end 112.395 113.2) (width 0.25) (layer F.Cu) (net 1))
 (segment (start 112.5625 114.1475) (end 112.395 113.98) (width 0.25) (layer F.Cu) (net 1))
 (segment (start 115.57 114.1475) (end 112.5625 114.1475) (width 0.25) (layer F.Cu) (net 1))
 (segment (start 115.7325 113.985) (end 115.57 114.1475) (width 0.25) (layer F.Cu) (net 1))
 (segment (start 117.475 113.985) (end 115.7325 113.985) (width 0.25) (layer F.Cu) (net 1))
 (segment (start 110.17 101.285) (end 110.49 100.965) (width 0.25) (layer F.Cu) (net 1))
 (segment (start 108.315 101.285) (end 110.17 101.285) (width 0.25) (layer F.Cu) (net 1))
 (segment (start 113.6675 115.7225) (end 113.345 115.4) (width 0.25) (layer F.Cu) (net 3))
 (segment (start 115.57 115.7225) (end 113.6675 115.7225) (width 0.25) (layer F.Cu) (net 3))
 (via (at 108.585 117.475) (size 1.7) (drill 1) (layers F.Cu B.Cu) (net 7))
 (segment (start 111.37 115.325) (end 111.445 115.4) (width 0.25) (layer F.Cu) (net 7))
 (segment (start 108.585 115.325) (end 111.37 115.325) (width 0.25) (layer F.Cu) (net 7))
 (segment (start 108.585 115.325) (end 108.585 117.475) (width 0.25) (layer F.Cu) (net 7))
 (segment (start 102.87 102.235) (end 102.235 101.6) (width 0.25) (layer F.Cu) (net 68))
 (segment (start 106.315 102.235) (end 102.87 102.235) (width 0.25) (layer F.Cu) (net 68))
 (segment (start 106.29 105.345) (end 106.29 106.045) (width 0.25) (layer F.Cu) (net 69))
 (segment (start 105.085 104.14) (end 106.29 105.345) (width 0.25) (layer F.Cu) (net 69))
 (segment (start 102.235 104.14) (end 105.085 104.14) (width 0.25) (layer F.Cu) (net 69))
 (segment (start 112.812499 118.650001) (end 112.8775 118.585) (width 0.25) (layer F.Cu) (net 72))
 (segment (start 108.020999 118.650001) (end 112.812499 118.650001) (width 0.25) (layer F.Cu) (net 72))
 (segment (start 105.44001 116.069012) (end 108.020999 118.650001) (width 0.25) (layer F.Cu) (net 72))
 (segment (start 105.44001 114.62501) (end 105.44001 116.069012) (width 0.25) (layer F.Cu) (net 72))
 (segment (start 112.8775 118.585) (end 112.8775 118.11) (width 0.25) (layer F.Cu) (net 72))
 (segment (start 105.115 114.3) (end 105.44001 114.62501) (width 0.25) (layer F.Cu) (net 72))
 (segment (start 104.14 114.3) (end 105.115 114.3) (width 0.25) (layer F.Cu) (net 72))
 (segment (start 112.44 120.015) (end 112.8775 120.015) (width 0.25) (layer F.Cu) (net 73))
 (segment (start 108.58 120.015) (end 112.44 120.015) (width 0.25) (layer F.Cu) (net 73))
 (segment (start 105.365 116.8) (end 108.58 120.015) (width 0.25) (layer F.Cu) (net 73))
 (segment (start 104.14 116.8) (end 105.365 116.8) (width 0.25) (layer F.Cu) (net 73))
 (segment (start 105.37 119.3) (end 108.625 122.555) (width 0.25) (layer F.Cu) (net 74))
 (segment (start 104.14 119.3) (end 105.37 119.3) (width 0.25) (layer F.Cu) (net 74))
 (segment (start 108.625 122.555) (end 113.625 122.555) (width 0.25) (layer F.Cu) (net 74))
 (segment (start 117.33 113.2) (end 117.475 113.345) (width 0.25) (layer F.Cu) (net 87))
 (segment (start 113.345 113.2) (end 117.33 113.2) (width 0.25) (layer F.Cu) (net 87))
 (segment (start 108.585 109.895) (end 108.625 109.855) (width 0.25) (layer F.Cu) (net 86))
 (segment (start 108.585 113.275) (end 108.585 109.895) (width 0.25) (layer F.Cu) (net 86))
 (segment (start 108.66 113.2) (end 108.585 113.275) (width 0.25) (layer F.Cu) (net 86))
 (segment (start 111.445 113.2) (end 108.66 113.2) (width 0.25) (layer F.Cu) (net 86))
 (segment (start 113.625 109.855) (end 108.625 109.855) (width 0.25) (layer F.Cu) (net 86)))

